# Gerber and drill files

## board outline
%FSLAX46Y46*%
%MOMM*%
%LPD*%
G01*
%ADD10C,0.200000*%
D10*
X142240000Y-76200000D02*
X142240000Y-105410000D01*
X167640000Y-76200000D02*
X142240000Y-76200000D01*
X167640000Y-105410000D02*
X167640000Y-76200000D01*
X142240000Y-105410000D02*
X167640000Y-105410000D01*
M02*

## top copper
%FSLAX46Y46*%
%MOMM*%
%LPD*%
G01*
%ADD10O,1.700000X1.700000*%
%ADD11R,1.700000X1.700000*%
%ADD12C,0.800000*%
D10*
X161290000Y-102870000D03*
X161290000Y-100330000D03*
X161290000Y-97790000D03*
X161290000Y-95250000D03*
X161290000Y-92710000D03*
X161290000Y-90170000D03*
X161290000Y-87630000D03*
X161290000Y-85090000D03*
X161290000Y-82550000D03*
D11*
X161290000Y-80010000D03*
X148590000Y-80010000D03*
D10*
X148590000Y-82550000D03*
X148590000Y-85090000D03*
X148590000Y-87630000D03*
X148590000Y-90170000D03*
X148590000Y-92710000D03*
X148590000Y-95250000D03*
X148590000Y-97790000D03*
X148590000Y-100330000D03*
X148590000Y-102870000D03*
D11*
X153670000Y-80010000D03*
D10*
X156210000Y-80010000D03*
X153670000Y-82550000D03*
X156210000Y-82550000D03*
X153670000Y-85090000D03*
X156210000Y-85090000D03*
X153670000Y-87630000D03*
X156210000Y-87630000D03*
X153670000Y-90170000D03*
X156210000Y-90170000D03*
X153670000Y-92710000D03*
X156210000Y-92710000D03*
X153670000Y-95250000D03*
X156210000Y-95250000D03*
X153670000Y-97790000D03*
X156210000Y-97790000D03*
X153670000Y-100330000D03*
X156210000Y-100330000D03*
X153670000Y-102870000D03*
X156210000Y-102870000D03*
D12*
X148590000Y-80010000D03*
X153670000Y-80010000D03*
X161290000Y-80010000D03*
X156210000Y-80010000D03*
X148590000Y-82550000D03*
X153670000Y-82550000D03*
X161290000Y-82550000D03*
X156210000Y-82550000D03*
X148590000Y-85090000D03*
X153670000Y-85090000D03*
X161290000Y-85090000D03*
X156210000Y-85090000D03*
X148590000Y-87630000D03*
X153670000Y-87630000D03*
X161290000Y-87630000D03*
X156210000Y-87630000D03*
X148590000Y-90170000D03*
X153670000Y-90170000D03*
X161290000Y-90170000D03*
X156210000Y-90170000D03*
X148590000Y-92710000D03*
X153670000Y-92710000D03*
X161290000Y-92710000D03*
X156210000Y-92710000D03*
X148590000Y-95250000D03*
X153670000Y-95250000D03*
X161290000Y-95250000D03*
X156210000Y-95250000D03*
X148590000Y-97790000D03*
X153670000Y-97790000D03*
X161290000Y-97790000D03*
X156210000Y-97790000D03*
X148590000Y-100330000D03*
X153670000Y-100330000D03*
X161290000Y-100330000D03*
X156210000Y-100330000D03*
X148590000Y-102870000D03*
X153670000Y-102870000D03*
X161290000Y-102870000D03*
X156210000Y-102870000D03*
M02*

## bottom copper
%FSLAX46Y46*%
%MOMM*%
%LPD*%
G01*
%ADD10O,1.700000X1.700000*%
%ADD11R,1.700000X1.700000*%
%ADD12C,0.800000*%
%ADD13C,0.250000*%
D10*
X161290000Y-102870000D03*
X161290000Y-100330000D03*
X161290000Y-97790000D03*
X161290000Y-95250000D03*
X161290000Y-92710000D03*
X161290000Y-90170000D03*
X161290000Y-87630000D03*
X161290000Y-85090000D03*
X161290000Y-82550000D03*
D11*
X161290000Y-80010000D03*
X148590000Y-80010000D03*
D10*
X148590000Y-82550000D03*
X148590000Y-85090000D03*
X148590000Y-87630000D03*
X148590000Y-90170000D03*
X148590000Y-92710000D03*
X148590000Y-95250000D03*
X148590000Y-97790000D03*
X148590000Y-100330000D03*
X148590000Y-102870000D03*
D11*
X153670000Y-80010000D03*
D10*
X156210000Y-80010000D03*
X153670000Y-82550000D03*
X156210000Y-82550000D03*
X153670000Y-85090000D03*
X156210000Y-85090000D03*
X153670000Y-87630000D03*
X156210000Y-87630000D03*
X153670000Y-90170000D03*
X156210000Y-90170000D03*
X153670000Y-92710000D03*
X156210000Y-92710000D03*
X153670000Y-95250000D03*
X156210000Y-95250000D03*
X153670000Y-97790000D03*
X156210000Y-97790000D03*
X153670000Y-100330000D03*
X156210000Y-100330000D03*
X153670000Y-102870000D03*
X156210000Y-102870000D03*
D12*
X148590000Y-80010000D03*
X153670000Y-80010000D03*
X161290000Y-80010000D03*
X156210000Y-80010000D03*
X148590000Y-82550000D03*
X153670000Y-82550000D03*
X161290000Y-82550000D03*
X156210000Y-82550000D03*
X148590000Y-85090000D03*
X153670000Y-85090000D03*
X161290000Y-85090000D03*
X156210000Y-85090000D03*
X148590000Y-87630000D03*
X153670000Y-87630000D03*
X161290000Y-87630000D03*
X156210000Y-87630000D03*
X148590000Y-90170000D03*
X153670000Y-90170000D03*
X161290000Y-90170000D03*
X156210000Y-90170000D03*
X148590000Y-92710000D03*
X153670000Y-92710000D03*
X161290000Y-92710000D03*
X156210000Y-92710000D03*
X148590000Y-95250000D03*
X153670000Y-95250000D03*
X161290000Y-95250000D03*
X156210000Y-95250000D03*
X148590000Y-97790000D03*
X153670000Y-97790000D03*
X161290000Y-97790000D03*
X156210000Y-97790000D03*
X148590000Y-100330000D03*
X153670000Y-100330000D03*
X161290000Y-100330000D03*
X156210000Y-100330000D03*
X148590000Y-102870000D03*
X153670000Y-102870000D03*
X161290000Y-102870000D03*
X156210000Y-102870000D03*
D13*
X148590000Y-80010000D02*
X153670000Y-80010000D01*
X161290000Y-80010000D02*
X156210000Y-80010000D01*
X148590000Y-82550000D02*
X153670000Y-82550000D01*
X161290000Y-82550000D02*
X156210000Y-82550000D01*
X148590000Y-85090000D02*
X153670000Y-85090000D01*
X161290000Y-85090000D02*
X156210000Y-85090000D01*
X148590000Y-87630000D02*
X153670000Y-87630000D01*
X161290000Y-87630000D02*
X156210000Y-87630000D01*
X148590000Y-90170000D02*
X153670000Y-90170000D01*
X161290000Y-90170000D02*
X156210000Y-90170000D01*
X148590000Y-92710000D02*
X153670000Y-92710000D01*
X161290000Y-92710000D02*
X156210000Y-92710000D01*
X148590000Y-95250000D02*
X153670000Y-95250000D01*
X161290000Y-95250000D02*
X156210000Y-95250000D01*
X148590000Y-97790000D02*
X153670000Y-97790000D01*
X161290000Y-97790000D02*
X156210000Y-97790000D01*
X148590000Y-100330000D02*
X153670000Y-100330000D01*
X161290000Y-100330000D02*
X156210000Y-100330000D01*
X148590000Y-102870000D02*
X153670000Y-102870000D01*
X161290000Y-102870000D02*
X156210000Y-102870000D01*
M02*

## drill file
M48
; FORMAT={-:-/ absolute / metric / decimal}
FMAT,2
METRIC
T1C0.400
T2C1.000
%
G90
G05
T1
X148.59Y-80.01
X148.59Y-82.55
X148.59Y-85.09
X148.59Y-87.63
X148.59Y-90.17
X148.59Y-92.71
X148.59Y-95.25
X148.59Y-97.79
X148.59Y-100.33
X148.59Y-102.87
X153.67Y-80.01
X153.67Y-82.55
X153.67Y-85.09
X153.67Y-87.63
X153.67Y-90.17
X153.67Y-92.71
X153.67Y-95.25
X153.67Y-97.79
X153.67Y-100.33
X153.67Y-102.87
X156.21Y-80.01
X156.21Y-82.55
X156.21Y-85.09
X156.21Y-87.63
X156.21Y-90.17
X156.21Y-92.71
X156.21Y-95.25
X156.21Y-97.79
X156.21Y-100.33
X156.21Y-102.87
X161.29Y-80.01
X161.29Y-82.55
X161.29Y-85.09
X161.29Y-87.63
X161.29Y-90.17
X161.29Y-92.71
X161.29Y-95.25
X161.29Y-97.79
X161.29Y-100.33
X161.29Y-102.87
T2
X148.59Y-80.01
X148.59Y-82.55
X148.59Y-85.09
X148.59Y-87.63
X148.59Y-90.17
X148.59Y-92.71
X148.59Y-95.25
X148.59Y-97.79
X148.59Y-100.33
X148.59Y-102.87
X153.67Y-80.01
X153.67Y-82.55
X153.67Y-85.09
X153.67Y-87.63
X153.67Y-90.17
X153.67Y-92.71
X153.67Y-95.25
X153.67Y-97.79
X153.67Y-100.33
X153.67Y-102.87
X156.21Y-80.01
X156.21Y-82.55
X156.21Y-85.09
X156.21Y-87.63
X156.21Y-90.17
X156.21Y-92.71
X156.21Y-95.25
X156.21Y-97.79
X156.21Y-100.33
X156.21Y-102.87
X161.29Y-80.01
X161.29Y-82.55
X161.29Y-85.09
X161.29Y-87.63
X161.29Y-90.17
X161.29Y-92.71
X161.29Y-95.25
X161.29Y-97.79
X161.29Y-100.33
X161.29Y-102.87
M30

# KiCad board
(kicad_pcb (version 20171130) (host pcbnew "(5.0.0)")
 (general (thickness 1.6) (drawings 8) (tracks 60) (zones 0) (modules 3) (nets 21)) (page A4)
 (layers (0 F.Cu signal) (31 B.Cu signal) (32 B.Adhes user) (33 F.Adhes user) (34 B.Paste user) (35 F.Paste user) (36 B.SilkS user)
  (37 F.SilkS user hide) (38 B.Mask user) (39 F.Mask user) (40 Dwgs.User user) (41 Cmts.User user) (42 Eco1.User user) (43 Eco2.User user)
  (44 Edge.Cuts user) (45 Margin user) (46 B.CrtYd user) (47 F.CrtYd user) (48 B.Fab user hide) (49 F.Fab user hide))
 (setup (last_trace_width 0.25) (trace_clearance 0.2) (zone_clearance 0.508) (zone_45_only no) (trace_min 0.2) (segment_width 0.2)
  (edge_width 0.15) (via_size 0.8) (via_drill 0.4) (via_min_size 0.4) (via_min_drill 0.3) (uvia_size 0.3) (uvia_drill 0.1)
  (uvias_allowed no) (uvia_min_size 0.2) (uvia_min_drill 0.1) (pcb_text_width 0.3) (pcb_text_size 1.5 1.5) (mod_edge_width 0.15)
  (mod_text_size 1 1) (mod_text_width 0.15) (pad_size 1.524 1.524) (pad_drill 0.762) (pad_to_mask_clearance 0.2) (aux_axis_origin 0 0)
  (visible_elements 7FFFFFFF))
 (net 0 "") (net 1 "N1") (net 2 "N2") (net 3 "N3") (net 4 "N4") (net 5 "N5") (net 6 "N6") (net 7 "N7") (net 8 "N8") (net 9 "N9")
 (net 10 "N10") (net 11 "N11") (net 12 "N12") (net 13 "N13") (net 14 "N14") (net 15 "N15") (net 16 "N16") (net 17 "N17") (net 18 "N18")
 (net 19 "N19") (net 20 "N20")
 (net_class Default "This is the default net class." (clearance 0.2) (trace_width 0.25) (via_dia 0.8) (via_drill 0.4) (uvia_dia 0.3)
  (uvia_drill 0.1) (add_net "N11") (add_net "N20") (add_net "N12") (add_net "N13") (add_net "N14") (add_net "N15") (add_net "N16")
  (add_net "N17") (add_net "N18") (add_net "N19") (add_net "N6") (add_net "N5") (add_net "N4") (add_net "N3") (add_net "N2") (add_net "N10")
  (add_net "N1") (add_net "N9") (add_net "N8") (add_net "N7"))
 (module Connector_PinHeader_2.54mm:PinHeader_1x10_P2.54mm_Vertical (layer F.Cu) (at 161.29 80.01)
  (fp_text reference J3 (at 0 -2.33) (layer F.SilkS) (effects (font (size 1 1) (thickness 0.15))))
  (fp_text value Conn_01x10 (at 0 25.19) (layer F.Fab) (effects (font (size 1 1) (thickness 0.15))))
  (pad 10 thru_hole oval (at 0 22.86) (size 1.7 1.7) (drill 1) (layers *.Cu *.Mask) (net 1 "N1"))
  (pad 9 thru_hole oval (at 0 20.32) (size 1.7 1.7) (drill 1) (layers *.Cu *.Mask) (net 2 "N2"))
  (pad 8 thru_hole oval (at 0 17.78) (size 1.7 1.7) (drill 1) (layers *.Cu *.Mask) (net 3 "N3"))
  (pad 7 thru_hole oval (at 0 15.24) (size 1.7 1.7) (drill 1) (layers *.Cu *.Mask) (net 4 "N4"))
  (pad 6 thru_hole oval (at 0 12.7) (size 1.7 1.7) (drill 1) (layers *.Cu *.Mask) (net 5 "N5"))
  (pad 5 thru_hole oval (at 0 10.16) (size 1.7 1.7) (drill 1) (layers *.Cu *.Mask) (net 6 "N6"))
  (pad 4 thru_hole oval (at 0 7.62) (size 1.7 1.7) (drill 1) (layers *.Cu *.Mask) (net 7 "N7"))
  (pad 3 thru_hole oval (at 0 5.08) (size 1.7 1.7) (drill 1) (layers *.Cu *.Mask) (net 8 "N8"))
  (pad 2 thru_hole oval (at 0 2.54) (size 1.7 1.7) (drill 1) (layers *.Cu *.Mask) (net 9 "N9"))
  (pad 1 thru_hole rect (at 0 0) (size 1.7 1.7) (drill 1) (layers *.Cu *.Mask) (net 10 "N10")))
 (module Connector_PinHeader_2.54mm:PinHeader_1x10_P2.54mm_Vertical (layer F.Cu) (at 148.59 80.01)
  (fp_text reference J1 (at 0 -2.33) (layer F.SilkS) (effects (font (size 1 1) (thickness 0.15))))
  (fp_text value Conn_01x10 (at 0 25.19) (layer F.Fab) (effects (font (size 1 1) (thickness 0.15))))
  (pad 1 thru_hole rect (at 0 0) (size 1.7 1.7) (drill 1) (layers *.Cu *.Mask) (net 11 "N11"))
  (pad 2 thru_hole oval (at 0 2.54) (size 1.7 1.7) (drill 1) (layers *.Cu *.Mask) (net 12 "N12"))
  (pad 3 thru_hole oval (at 0 5.08) (size 1.7 1.7) (drill 1) (layers *.Cu *.Mask) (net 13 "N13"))
  (pad 4 thru_hole oval (at 0 7.62) (size 1.7 1.7) (drill 1) (layers *.Cu *.Mask) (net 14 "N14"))
  (pad 5 thru_hole oval (at 0 10.16) (size 1.7 1.7) (drill 1) (layers *.Cu *.Mask) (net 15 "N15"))
  (pad 6 thru_hole oval (at 0 12.7) (size 1.7 1.7) (drill 1) (layers *.Cu *.Mask) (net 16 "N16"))
  (pad 7 thru_hole oval (at 0 15.24) (size 1.7 1.7) (drill 1) (layers *.Cu *.Mask) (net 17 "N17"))
  (pad 8 thru_hole oval (at 0 17.78) (size 1.7 1.7) (drill 1) (layers *.Cu *.Mask) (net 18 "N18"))
  (pad 9 thru_hole oval (at 0 20.32) (size 1.7 1.7) (drill 1) (layers *.Cu *.Mask) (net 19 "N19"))
  (pad 10 thru_hole oval (at 0 22.86) (size 1.7 1.7) (drill 1) (layers *.Cu *.Mask) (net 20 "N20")))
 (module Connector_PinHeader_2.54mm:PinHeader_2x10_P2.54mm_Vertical (layer F.Cu) (at 153.67 80.01)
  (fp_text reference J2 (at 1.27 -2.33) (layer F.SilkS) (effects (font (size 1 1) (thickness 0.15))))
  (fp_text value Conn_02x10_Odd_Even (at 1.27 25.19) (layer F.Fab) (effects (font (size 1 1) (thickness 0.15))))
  (pad 1 thru_hole rect (at 0 0) (size 1.7 1.7) (drill 1) (layers *.Cu *.Mask) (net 11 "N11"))
  (pad 2 thru_hole oval (at 2.54 0) (size 1.7 1.7) (drill 1) (layers *.Cu *.Mask) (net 10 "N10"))
  (pad 3 thru_hole oval (at 0 2.54) (size 1.7 1.7) (drill 1) (layers *.Cu *.Mask) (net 12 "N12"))
  (pad 4 thru_hole oval (at 2.54 2.54) (size 1.7 1.7) (drill 1) (layers *.Cu *.Mask) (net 9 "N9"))
  (pad 5 thru_hole oval (at 0 5.08) (size 1.7 1.7) (drill 1) (layers *.Cu *.Mask) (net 13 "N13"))
  (pad 6 thru_hole oval (at 2.54 5.08) (size 1.7 1.7) (drill 1) (layers *.Cu *.Mask) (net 8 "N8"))
  (pad 7 thru_hole oval (at 0 7.62) (size 1.7 1.7) (drill 1) (layers *.Cu *.Mask) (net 14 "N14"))
  (pad 8 thru_hole oval (at 2.54 7.62) (size 1.7 1.7) (drill 1) (layers *.Cu *.Mask) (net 7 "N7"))
  (pad 9 thru_hole oval (at 0 10.16) (size 1.7 1.7) (drill 1) (layers *.Cu *.Mask) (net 15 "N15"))
  (pad 10 thru_hole oval (at 2.54 10.16) (size 1.7 1.7) (drill 1) (layers *.Cu *.Mask) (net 6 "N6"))
  (pad 11 thru_hole oval (at 0 12.7) (size 1.7 1.7) (drill 1) (layers *.Cu *.Mask) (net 16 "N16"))
  (pad 12 thru_hole oval (at 2.54 12.7) (size 1.7 1.7) (drill 1) (layers *.Cu *.Mask) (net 5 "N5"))
  (pad 13 thru_hole oval (at 0 15.24) (size 1.7 1.7) (drill 1) (layers *.Cu *.Mask) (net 17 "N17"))
  (pad 14 thru_hole oval (at 2.54 15.24) (size 1.7 1.7) (drill 1) (layers *.Cu *.Mask) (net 4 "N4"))
  (pad 15 thru_hole oval (at 0 17.78) (size 1.7 1.7) (drill 1) (layers *.Cu *.Mask) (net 18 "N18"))
  (pad 16 thru_hole oval (at 2.54 17.78) (size 1.7 1.7) (drill 1) (layers *.Cu *.Mask) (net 3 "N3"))
  (pad 17 thru_hole oval (at 0 20.32) (size 1.7 1.7) (drill 1) (layers *.Cu *.Mask) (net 19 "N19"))
  (pad 18 thru_hole oval (at 2.54 20.32) (size 1.7 1.7) (drill 1) (layers *.Cu *.Mask) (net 2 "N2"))
  (pad 19 thru_hole oval (at 0 22.86) (size 1.7 1.7) (drill 1) (layers *.Cu *.Mask) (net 20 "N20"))
  (pad 20 thru_hole oval (at 2.54 22.86) (size 1.7 1.7) (drill 1) (layers *.Cu *.Mask) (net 1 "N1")))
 (gr_line (start 142.24 76.2) (end 142.24 105.41) (layer Edge.Cuts) (width 0.2))
 (gr_line (start 167.64 76.2) (end 142.24 76.2) (layer Edge.Cuts) (width 0.2))
 (gr_line (start 167.64 105.41) (end 167.64 76.2) (layer Edge.Cuts) (width 0.2))
 (gr_line (start 142.24 105.41) (end 167.64 105.41) (layer Edge.Cuts) (width 0.2))
 (segment (start 148.59 80.01) (end 153.67 80.01) (width 0.25) (layer B.Cu) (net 11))
 (via (at 148.59 80.01) (size 0.8) (layers F.Cu B.Cu) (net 11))
 (via (at 153.67 80.01) (size 0.8) (layers F.Cu B.Cu) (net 11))
 (segment (start 161.29 80.01) (end 156.21 80.01) (width 0.25) (layer B.Cu) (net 10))
 (via (at 161.29 80.01) (size 0.8) (layers F.Cu B.Cu) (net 10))
 (via (at 156.21 80.01) (size 0.8) (layers F.Cu B.Cu) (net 10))
 (segment (start 148.59 82.55) (end 153.67 82.55) (width 0.25) (layer B.Cu) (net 12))
 (via (at 148.59 82.55) (size 0.8) (layers F.Cu B.Cu) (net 12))
 (via (at 153.67 82.55) (size 0.8) (layers F.Cu B.Cu) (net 12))
 (segment (start 161.29 82.55) (end 156.21 82.55) (width 0.25) (layer B.Cu) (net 9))
 (via (at 161.29 82.55) (size 0.8) (layers F.Cu B.Cu) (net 9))
 (via (at 156.21 82.55) (size 0.8) (layers F.Cu B.Cu) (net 9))
 (segment (start 148.59 85.09) (end 153.67 85.09) (width 0.25) (layer B.Cu) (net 13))
 (via (at 148.59 85.09) (size 0.8) (layers F.Cu B.Cu) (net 13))
 (via (at 153.67 85.09) (size 0.8) (layers F.Cu B.Cu) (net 13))
 (segment (start 161.29 85.09) (end 156.21 85.09) (width 0.25) (layer B.Cu) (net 8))
 (via (at 161.29 85.09) (size 0.8) (layers F.Cu B.Cu) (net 8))
 (via (at 156.21 85.09) (size 0.8) (layers F.Cu B.Cu) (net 8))
 (segment (start 148.59 87.63) (end 153.67 87.63) (width 0.25) (layer B.Cu) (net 14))
 (via (at 148.59 87.63) (size 0.8) (layers F.Cu B.Cu) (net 14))
 (via (at 153.67 87.63) (size 0.8) (layers F.Cu B.Cu) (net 14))
 (segment (start 161.29 87.63) (end 156.21 87.63) (width 0.25) (layer B.Cu) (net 7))
 (via (at 161.29 87.63) (size 0.8) (layers F.Cu B.Cu) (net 7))
 (via (at 156.21 87.63) (size 0.8) (layers F.Cu B.Cu) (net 7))
 (segment (start 148.59 90.17) (end 153.67 90.17) (width 0.25) (layer B.Cu) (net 15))
 (via (at 148.59 90.17) (size 0.8) (layers F.Cu B.Cu) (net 15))
 (via (at 153.67 90.17) (size 0.8) (layers F.Cu B.Cu) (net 15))
 (segment (start 161.29 90.17) (end 156.21 90.17) (width 0.25) (layer B.Cu) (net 6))
 (via (at 161.29 90.17) (size 0.8) (layers F.Cu B.Cu) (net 6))
 (via (at 156.21 90.17) (size 0.8) (layers F.Cu B.Cu) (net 6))
 (segment (start 148.59 92.71) (end 153.67 92.71) (width 0.25) (layer B.Cu) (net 16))
 (via (at 148.59 92.71) (size 0.8) (layers F.Cu B.Cu) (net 16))
 (via (at 153.67 92.71) (size 0.8) (layers F.Cu B.Cu) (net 16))
 (segment (start 161.29 92.71) (end 156.21 92.71) (width 0.25) (layer B.Cu) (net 5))
 (via (at 161.29 92.71) (size 0.8) (layers F.Cu B.Cu) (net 5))
 (via (at 156.21 92.71) (size 0.8) (layers F.Cu B.Cu) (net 5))
 (segment (start 148.59 95.25) (end 153.67 95.25) (width 0.25) (layer B.Cu) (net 17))
 (via (at 148.59 95.25) (size 0.8) (layers F.Cu B.Cu) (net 17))
 (via (at 153.67 95.25) (size 0.8) (layers F.Cu B.Cu) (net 17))
 (segment (start 161.29 95.25) (end 156.21 95.25) (width 0.25) (layer B.Cu) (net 4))
 (via (at 161.29 95.25) (size 0.8) (layers F.Cu B.Cu) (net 4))
 (via (at 156.21 95.25) (size 0.8) (layers F.Cu B.Cu) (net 4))
 (segment (start 148.59 97.79) (end 153.67 97.79) (width 0.25) (layer B.Cu) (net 18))
 (via (at 148.59 97.79) (size 0.8) (layers F.Cu B.Cu) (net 18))
 (via (at 153.67 97.79) (size 0.8) (layers F.Cu B.Cu) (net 18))
 (segment (start 161.29 97.79) (end 156.21 97.79) (width 0.25) (layer B.Cu) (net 3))
 (via (at 161.29 97.79) (size 0.8) (layers F.Cu B.Cu) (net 3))
 (via (at 156.21 97.79) (size 0.8) (layers F.Cu B.Cu) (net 3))
 (segment (start 148.59 100.33) (end 153.67 100.33) (width 0.25) (layer B.Cu) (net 19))
 (via (at 148.59 100.33) (size 0.8) (layers F.Cu B.Cu) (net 19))
 (via (at 153.67 100.33) (size 0.8) (layers F.Cu B.Cu) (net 19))
 (segment (start 161.29 100.33) (end 156.21 100.33) (width 0.25) (layer B.Cu) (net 2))
 (via (at 161.29 100.33) (size 0.8) (layers F.Cu B.Cu) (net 2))
 (via (at 156.21 100.33) (size 0.8) (layers F.Cu B.Cu) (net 2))
 (segment (start 148.59 102.87) (end 153.67 102.87) (width 0.25) (layer B.Cu) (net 20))
 (via (at 148.59 102.87) (size 0.8) (layers F.Cu B.Cu) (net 20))
 (via (at 153.67 102.87) (size 0.8) (layers F.Cu B.Cu) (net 20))
 (segment (start 161.29 102.87) (end 156.21 102.87) (width 0.25) (layer B.Cu) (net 1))
 (via (at 161.29 102.87) (size 0.8) (layers F.Cu B.Cu) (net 1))
 (via (at 156.21 102.87) (size 0.8) (layers F.Cu B.Cu) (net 1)))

